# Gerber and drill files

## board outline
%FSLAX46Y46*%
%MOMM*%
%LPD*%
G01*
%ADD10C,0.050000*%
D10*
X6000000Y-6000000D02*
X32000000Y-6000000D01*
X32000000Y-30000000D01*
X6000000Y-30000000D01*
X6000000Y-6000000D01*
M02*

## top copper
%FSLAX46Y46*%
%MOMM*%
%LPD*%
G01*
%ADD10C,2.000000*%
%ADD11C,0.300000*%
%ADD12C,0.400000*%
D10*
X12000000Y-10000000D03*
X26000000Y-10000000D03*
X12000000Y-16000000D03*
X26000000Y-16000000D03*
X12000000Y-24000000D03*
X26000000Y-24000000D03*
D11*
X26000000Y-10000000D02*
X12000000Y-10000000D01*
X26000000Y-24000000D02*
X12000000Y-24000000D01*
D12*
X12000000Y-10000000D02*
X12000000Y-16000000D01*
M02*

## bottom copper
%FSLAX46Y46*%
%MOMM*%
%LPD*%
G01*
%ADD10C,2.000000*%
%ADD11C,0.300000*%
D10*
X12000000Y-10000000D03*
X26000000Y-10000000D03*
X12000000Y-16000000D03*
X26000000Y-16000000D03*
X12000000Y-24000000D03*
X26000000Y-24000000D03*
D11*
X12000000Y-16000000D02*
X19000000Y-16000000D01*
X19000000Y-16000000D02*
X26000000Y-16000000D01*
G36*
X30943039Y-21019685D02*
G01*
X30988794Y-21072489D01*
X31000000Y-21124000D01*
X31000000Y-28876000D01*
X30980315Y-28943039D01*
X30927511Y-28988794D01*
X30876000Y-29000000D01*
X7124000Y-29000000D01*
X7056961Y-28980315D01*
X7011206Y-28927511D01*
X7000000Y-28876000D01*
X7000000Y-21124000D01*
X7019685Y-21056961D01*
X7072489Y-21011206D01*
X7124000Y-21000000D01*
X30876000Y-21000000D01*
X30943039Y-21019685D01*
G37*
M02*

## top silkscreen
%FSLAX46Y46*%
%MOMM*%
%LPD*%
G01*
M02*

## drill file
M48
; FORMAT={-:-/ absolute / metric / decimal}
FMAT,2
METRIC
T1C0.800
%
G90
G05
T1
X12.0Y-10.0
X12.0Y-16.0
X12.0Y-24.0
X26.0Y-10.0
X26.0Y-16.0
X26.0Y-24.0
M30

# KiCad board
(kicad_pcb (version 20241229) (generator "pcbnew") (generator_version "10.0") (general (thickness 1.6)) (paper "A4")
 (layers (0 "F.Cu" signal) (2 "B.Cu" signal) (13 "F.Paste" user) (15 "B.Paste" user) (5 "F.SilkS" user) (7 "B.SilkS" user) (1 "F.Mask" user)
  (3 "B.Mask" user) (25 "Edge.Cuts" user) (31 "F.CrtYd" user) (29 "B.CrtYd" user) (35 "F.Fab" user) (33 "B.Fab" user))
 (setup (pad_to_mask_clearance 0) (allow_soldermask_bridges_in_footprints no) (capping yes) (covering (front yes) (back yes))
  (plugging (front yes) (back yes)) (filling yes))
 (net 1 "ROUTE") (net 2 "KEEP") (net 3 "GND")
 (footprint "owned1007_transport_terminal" (layer "F.Cu") (at 12 10)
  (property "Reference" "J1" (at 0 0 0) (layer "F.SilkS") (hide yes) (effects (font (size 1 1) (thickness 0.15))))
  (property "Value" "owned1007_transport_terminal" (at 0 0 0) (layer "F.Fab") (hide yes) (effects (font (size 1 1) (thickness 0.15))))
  (pad "1" thru_hole circle (at 0 0) (size 2 2) (drill 0.8) (layers "*.Cu" "*.Mask") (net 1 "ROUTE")))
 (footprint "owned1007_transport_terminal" (layer "F.Cu") (at 26 10)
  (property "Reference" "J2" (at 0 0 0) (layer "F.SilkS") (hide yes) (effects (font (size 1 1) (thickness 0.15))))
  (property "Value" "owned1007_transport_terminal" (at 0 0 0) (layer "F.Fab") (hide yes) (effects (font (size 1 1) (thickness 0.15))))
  (pad "1" thru_hole circle (at 0 0) (size 2 2) (drill 0.8) (layers "*.Cu" "*.Mask") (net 1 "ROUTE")))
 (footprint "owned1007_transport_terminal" (layer "F.Cu") (at 12 16)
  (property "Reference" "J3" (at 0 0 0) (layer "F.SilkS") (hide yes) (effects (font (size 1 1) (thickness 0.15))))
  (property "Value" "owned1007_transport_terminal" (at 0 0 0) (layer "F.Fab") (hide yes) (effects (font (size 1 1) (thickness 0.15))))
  (pad "1" thru_hole circle (at 0 0) (size 2 2) (drill 0.8) (layers "*.Cu" "*.Mask") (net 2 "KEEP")))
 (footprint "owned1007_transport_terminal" (layer "F.Cu") (at 26 16)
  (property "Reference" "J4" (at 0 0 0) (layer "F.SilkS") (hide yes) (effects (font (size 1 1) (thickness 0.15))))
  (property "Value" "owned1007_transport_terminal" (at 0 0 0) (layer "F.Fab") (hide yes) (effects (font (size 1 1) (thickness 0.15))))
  (pad "1" thru_hole circle (at 0 0) (size 2 2) (drill 0.8) (layers "*.Cu" "*.Mask") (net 2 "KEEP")))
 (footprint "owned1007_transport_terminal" (layer "F.Cu") (at 12 24)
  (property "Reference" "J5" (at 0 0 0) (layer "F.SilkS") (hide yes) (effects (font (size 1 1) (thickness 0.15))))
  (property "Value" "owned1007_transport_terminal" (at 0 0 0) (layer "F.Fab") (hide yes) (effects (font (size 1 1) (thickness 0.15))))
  (pad "1" thru_hole circle (at 0 0) (size 2 2) (drill 0.8) (layers "*.Cu" "*.Mask") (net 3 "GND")))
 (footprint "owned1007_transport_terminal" (layer "F.Cu") (at 26 24)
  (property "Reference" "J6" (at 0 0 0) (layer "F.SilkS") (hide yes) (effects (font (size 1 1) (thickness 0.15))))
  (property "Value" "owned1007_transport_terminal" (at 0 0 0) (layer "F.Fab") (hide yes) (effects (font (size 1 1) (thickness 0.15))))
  (pad "1" thru_hole circle (at 0 0) (size 2 2) (drill 0.8) (layers "*.Cu" "*.Mask") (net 3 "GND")))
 (gr_rect (start 6 6) (end 32 30) (stroke (width 0.05) (type default)) (fill none) (layer "Edge.Cuts"))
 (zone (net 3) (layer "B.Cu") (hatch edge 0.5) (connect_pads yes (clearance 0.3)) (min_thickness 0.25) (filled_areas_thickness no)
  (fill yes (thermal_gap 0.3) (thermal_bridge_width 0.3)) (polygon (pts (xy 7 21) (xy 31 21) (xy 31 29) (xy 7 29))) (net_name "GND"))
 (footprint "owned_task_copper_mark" (layer "F.Cu") (at 10 28)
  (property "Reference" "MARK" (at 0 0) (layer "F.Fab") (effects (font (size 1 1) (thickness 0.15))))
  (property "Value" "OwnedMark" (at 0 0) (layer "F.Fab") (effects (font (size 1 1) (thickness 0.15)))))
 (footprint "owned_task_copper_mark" (layer "F.Cu") (at 13 28)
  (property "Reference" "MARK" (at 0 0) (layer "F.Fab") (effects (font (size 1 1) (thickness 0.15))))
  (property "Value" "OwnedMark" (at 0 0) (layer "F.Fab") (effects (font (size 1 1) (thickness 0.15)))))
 (segment (start 26 10) (end 12 10) (width 0.3) (layer "F.Cu") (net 1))
 (segment (start 12 16) (end 19 16) (width 0.3) (layer "B.Cu") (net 2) (locked yes))
 (segment (start 19 16) (end 26 16) (width 0.3) (layer "B.Cu") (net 2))
 (segment (start 26 24) (end 12 24) (width 0.3) (layer "F.Cu") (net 3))
 (segment (start 12 10) (end 12 16) (width 0.4) (layer "F.Cu") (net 1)))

